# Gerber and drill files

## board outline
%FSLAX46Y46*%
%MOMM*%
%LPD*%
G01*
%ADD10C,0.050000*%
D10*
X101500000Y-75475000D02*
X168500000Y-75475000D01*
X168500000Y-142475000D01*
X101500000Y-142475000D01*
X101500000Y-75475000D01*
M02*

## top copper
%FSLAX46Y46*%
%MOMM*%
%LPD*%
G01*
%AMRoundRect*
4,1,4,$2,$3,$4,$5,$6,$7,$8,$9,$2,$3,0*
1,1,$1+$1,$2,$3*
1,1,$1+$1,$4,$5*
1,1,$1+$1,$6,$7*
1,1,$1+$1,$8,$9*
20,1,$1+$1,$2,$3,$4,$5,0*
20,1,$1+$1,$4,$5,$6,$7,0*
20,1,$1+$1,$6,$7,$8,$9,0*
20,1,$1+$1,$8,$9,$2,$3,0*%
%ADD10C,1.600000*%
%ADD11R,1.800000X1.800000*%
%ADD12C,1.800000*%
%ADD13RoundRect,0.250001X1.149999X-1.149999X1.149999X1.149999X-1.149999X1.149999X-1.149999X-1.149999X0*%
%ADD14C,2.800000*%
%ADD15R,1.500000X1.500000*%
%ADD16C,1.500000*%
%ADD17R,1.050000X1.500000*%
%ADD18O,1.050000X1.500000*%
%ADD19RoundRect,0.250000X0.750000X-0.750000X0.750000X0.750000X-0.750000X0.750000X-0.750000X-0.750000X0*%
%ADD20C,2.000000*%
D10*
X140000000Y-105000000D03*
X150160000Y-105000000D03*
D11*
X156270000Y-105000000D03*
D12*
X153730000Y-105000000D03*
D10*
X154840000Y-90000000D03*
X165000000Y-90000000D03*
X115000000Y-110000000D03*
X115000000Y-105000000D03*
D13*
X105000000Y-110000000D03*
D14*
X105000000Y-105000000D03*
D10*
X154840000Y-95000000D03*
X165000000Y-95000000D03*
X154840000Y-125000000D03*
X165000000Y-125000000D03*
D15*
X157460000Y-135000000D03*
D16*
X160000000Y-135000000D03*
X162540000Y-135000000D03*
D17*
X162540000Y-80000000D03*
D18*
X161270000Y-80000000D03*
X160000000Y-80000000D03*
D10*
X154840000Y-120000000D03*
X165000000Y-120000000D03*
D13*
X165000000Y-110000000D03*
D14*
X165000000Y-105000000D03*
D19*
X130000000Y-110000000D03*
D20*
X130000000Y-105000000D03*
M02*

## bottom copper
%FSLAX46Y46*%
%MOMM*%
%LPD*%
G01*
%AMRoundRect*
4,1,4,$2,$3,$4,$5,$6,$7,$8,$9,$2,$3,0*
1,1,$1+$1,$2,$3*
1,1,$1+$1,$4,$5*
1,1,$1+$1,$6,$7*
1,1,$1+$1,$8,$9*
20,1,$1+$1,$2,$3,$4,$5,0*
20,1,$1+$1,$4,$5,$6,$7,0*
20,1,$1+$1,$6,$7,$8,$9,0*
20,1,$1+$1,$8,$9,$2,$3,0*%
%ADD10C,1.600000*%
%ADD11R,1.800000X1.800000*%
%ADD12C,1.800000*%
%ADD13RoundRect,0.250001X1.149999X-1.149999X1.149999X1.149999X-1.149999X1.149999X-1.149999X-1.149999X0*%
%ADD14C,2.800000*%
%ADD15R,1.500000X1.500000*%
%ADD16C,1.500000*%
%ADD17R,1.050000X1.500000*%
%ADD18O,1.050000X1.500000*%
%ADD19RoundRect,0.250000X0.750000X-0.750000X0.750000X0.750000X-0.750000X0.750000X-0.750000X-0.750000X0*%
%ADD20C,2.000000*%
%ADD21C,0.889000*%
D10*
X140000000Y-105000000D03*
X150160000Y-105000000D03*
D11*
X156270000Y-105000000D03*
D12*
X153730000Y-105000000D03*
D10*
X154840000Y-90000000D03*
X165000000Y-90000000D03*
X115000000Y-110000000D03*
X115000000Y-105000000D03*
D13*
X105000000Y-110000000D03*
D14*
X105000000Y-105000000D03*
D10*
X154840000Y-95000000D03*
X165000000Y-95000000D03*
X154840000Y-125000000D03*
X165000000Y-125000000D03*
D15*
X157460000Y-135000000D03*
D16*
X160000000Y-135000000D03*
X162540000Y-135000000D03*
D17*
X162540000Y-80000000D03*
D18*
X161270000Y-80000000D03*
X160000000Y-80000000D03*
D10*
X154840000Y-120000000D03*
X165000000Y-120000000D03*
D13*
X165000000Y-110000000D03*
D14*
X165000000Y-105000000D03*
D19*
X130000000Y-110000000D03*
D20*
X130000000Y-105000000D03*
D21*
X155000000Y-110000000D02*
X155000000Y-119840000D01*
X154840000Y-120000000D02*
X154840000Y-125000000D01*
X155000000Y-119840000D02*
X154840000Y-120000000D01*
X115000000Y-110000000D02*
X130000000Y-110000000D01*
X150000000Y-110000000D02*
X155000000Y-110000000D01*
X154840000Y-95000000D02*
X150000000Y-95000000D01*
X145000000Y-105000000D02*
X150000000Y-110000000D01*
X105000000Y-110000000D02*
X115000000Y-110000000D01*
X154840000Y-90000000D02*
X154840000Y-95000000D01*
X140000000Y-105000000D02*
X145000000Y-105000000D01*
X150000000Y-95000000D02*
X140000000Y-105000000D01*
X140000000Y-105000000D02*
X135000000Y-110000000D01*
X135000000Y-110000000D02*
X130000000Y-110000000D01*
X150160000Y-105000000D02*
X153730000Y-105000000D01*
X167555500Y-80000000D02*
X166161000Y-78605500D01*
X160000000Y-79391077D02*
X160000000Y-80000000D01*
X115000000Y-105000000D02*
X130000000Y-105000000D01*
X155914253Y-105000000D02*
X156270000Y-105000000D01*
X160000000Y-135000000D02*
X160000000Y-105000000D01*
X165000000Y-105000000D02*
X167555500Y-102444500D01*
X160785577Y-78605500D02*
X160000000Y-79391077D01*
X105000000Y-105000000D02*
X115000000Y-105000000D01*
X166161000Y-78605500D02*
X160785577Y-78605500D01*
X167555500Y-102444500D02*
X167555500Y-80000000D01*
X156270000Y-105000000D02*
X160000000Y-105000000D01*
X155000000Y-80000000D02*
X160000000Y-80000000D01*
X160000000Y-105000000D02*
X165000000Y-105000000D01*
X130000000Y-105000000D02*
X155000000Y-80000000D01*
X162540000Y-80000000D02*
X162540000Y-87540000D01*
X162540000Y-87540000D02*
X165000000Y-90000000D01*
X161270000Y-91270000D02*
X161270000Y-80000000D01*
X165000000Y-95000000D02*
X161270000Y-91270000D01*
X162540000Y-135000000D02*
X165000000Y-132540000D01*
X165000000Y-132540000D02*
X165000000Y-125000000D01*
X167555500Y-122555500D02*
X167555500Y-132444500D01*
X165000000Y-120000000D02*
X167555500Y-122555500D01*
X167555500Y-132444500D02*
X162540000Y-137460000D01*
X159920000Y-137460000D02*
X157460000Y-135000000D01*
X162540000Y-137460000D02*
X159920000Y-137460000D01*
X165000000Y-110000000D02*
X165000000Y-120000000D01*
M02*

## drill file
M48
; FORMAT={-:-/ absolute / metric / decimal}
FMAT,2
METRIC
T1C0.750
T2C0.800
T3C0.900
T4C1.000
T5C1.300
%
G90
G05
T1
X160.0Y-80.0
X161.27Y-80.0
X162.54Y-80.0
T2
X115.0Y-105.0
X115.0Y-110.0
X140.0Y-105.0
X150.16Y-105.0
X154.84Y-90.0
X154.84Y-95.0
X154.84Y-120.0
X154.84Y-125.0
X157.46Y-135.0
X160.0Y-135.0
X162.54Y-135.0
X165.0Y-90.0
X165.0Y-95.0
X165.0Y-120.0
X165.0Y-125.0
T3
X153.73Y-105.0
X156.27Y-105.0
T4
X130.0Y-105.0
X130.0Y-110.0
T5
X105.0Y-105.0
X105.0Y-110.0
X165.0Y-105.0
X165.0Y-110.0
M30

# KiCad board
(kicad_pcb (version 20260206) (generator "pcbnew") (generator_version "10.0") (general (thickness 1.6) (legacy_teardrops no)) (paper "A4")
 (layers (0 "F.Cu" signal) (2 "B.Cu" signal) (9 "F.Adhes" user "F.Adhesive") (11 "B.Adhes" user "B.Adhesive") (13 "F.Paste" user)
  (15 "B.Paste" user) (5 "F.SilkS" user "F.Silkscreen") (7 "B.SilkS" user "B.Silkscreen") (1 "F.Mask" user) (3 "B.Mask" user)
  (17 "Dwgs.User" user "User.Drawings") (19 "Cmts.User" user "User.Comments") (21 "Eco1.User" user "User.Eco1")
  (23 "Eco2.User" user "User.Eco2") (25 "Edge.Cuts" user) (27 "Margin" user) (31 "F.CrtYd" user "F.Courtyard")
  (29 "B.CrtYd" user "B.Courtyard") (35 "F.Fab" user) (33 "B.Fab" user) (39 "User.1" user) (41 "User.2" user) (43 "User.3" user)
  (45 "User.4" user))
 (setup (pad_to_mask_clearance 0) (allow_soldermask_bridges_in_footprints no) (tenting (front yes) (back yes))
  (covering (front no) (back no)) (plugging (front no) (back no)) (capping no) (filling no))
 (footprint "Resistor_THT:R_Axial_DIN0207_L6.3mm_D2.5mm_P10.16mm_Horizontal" (layer "F.Cu") (at 140 105)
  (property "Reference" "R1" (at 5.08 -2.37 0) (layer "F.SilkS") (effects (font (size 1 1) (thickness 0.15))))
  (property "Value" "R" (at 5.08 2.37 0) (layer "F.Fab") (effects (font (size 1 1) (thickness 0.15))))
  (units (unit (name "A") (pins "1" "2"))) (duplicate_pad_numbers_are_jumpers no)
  (pad "1" thru_hole circle (at 0 0) (size 1.6 1.6) (drill 0.8) (layers "*.Cu" "*.Mask") (remove_unused_layers no) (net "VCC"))
  (pad "2" thru_hole circle (at 10.16 0) (size 1.6 1.6) (drill 0.8) (layers "*.Cu" "*.Mask") (remove_unused_layers no) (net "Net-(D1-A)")))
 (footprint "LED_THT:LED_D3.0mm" (layer "F.Cu") (at 156.27 105 180)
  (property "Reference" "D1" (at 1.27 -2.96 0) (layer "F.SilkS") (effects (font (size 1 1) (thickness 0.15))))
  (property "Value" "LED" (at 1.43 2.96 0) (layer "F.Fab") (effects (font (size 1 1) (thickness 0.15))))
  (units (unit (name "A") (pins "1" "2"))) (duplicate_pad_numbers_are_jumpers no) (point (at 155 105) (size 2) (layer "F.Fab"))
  (pad "1" thru_hole rect (at 0 0 180) (size 1.8 1.8) (drill 0.9) (layers "*.Cu" "*.Mask") (remove_unused_layers no) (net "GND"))
  (pad "2" thru_hole circle (at 2.54 0 180) (size 1.8 1.8) (drill 0.9) (layers "*.Cu" "*.Mask") (remove_unused_layers no) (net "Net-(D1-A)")))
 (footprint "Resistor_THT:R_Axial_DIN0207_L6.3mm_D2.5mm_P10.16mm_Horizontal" (layer "F.Cu") (at 154.84 90)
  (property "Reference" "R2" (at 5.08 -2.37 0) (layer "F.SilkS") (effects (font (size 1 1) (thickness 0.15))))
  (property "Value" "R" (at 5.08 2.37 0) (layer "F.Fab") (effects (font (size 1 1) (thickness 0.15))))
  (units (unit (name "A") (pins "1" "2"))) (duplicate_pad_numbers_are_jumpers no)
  (pad "1" thru_hole circle (at 0 0) (size 1.6 1.6) (drill 0.8) (layers "*.Cu" "*.Mask") (remove_unused_layers no) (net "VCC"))
  (pad "2" thru_hole circle (at 10.16 0) (size 1.6 1.6) (drill 0.8) (layers "*.Cu" "*.Mask") (remove_unused_layers no) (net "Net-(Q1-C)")))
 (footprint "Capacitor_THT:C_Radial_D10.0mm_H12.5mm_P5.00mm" (layer "F.Cu") (at 115 110 90)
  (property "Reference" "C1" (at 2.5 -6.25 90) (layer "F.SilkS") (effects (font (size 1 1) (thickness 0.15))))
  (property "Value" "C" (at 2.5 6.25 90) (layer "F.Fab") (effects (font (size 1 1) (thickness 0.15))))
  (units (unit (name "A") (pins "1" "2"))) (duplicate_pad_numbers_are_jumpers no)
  (pad "1" thru_hole circle (at 0 0 90) (size 1.6 1.6) (drill 0.8) (layers "*.Cu" "*.Mask") (remove_unused_layers no) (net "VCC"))
  (pad "2" thru_hole circle (at 5 0 90) (size 1.6 1.6) (drill 0.8) (layers "*.Cu" "*.Mask") (remove_unused_layers no) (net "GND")))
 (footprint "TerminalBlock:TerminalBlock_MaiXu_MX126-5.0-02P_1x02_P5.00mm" (layer "F.Cu") (at 105 110 90)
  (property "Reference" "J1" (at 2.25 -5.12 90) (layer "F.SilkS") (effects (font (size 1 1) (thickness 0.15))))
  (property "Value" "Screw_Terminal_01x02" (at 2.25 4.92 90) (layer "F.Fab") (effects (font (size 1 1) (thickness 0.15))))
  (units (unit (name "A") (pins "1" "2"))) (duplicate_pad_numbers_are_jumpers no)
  (pad "1" thru_hole roundrect (at 0 0 90) (size 2.8 2.8) (drill 1.3) (layers "*.Cu" "*.Mask") (remove_unused_layers no)
   (roundrect_rratio 0.089286) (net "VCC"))
  (pad "2" thru_hole circle (at 5 0 90) (size 2.8 2.8) (drill 1.3) (layers "*.Cu" "*.Mask") (remove_unused_layers no) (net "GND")))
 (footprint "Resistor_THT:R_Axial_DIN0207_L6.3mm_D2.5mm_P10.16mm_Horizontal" (layer "F.Cu") (at 154.84 95)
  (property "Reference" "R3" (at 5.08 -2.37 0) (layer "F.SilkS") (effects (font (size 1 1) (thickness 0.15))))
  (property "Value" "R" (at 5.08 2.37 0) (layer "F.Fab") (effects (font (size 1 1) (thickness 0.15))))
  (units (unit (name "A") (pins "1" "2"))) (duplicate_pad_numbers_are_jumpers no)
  (pad "1" thru_hole circle (at 0 0) (size 1.6 1.6) (drill 0.8) (layers "*.Cu" "*.Mask") (remove_unused_layers no) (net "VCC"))
  (pad "2" thru_hole circle (at 10.16 0) (size 1.6 1.6) (drill 0.8) (layers "*.Cu" "*.Mask") (remove_unused_layers no) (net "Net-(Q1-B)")))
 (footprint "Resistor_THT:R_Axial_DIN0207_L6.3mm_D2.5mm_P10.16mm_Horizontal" (layer "F.Cu") (at 154.84 125)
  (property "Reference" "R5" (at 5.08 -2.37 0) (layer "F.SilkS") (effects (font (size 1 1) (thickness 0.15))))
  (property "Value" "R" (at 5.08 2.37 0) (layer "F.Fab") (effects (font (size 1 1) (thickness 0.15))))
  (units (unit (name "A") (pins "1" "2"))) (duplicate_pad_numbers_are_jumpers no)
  (pad "1" thru_hole circle (at 0 0) (size 1.6 1.6) (drill 0.8) (layers "*.Cu" "*.Mask") (remove_unused_layers no) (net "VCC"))
  (pad "2" thru_hole circle (at 10.16 0) (size 1.6 1.6) (drill 0.8) (layers "*.Cu" "*.Mask") (remove_unused_layers no) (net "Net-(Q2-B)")))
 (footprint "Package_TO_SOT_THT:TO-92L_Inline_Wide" (layer "F.Cu") (at 157.46 135)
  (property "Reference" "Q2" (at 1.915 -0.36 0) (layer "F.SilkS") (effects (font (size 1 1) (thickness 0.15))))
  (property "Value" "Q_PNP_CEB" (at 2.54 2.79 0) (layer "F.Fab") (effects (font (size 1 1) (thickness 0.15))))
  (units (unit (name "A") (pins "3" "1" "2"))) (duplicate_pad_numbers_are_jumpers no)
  (pad "1" thru_hole rect (at 0 0) (size 1.5 1.5) (drill 0.8) (layers "*.Cu" "*.Mask") (remove_unused_layers no) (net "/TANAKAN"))
  (pad "2" thru_hole circle (at 2.54 0) (size 1.5 1.5) (drill 0.8) (layers "*.Cu" "*.Mask") (remove_unused_layers no) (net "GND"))
  (pad "3" thru_hole circle (at 5.08 0) (size 1.5 1.5) (drill 0.8) (layers "*.Cu" "*.Mask") (remove_unused_layers no) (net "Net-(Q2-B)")))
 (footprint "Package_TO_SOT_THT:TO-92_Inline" (layer "F.Cu") (at 162.54 80 180)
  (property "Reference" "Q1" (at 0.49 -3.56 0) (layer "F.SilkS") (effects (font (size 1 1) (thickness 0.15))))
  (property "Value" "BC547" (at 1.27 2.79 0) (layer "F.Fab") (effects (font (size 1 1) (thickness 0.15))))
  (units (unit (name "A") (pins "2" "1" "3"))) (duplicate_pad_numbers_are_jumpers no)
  (pad "1" thru_hole rect (at 0 0 180) (size 1.05 1.5) (drill 0.75) (layers "*.Cu" "*.Mask") (remove_unused_layers no) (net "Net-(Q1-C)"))
  (pad "2" thru_hole oval (at 1.27 0 180) (size 1.05 1.5) (drill 0.75) (layers "*.Cu" "*.Mask") (remove_unused_layers no) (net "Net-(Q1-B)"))
  (pad "3" thru_hole oval (at 2.54 0 180) (size 1.05 1.5) (drill 0.75) (layers "*.Cu" "*.Mask") (remove_unused_layers no) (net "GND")))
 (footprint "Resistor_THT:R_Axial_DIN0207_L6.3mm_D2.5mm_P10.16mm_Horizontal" (layer "F.Cu") (at 154.84 120)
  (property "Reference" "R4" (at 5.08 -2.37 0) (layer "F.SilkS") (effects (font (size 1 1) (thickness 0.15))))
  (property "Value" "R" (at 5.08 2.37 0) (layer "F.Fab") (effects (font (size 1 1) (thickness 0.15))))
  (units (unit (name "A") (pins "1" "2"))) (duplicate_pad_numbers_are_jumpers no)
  (pad "1" thru_hole circle (at 0 0) (size 1.6 1.6) (drill 0.8) (layers "*.Cu" "*.Mask") (remove_unused_layers no) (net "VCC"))
  (pad "2" thru_hole circle (at 10.16 0) (size 1.6 1.6) (drill 0.8) (layers "*.Cu" "*.Mask") (remove_unused_layers no) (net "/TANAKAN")))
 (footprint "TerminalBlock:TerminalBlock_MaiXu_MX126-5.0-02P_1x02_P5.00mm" (layer "F.Cu") (at 165 110 90)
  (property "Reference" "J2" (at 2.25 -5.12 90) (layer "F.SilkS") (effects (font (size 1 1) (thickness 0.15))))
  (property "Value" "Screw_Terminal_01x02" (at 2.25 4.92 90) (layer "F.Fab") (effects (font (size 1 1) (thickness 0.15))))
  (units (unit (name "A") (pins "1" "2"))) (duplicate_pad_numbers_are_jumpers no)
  (pad "1" thru_hole roundrect (at 0 0 90) (size 2.8 2.8) (drill 1.3) (layers "*.Cu" "*.Mask") (remove_unused_layers no)
   (roundrect_rratio 0.089286) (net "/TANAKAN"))
  (pad "2" thru_hole circle (at 5 0 90) (size 2.8 2.8) (drill 1.3) (layers "*.Cu" "*.Mask") (remove_unused_layers no) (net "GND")))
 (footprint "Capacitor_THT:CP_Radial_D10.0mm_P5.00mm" (layer "F.Cu") (at 130 110 90)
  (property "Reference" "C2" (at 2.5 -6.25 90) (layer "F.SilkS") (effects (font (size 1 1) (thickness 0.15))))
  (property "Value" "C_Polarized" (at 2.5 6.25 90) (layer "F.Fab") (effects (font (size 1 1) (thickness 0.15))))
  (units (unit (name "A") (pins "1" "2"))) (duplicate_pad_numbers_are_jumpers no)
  (pad "1" thru_hole roundrect (at 0 0 90) (size 2 2) (drill 1) (layers "*.Cu" "*.Mask") (remove_unused_layers no) (roundrect_rratio 0.125)
   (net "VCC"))
  (pad "2" thru_hole circle (at 5 0 90) (size 2 2) (drill 1) (layers "*.Cu" "*.Mask") (remove_unused_layers no) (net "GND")))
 (gr_rect (start 101.5 75.475) (end 168.5 142.475) (stroke (width 0.05) (type default)) (fill no) (layer "Edge.Cuts"))
 (segment (start 155 110) (end 155 119.84) (width 0.889) (layer "B.Cu") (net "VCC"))
 (segment (start 154.84 120) (end 154.84 125) (width 0.889) (layer "B.Cu") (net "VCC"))
 (segment (start 155 119.84) (end 154.84 120) (width 0.889) (layer "B.Cu") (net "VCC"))
 (segment (start 115 110) (end 130 110) (width 0.889) (layer "B.Cu") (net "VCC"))
 (segment (start 150 110) (end 155 110) (width 0.889) (layer "B.Cu") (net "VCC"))
 (segment (start 154.84 95) (end 150 95) (width 0.889) (layer "B.Cu") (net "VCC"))
 (segment (start 145 105) (end 150 110) (width 0.889) (layer "B.Cu") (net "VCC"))
 (segment (start 105 110) (end 115 110) (width 0.889) (layer "B.Cu") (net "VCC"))
 (segment (start 154.84 90) (end 154.84 95) (width 0.889) (layer "B.Cu") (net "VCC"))
 (segment (start 140 105) (end 145 105) (width 0.889) (layer "B.Cu") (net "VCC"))
 (segment (start 150 95) (end 140 105) (width 0.889) (layer "B.Cu") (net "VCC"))
 (segment (start 140 105) (end 135 110) (width 0.889) (layer "B.Cu") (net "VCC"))
 (segment (start 135 110) (end 130 110) (width 0.889) (layer "B.Cu") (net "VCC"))
 (segment (start 150.16 105) (end 153.73 105) (width 0.889) (layer "B.Cu") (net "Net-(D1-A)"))
 (segment (start 167.5555 80) (end 166.161 78.6055) (width 0.889) (layer "B.Cu") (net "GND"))
 (segment (start 160 79.391077) (end 160 80) (width 0.889) (layer "B.Cu") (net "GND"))
 (segment (start 115 105) (end 130 105) (width 0.889) (layer "B.Cu") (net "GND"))
 (segment (start 155.914253 105) (end 156.27 105) (width 0.889) (layer "B.Cu") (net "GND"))
 (segment (start 160 135) (end 160 105) (width 0.889) (layer "B.Cu") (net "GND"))
 (segment (start 165 105) (end 167.5555 102.4445) (width 0.889) (layer "B.Cu") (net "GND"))
 (segment (start 160.785577 78.6055) (end 160 79.391077) (width 0.889) (layer "B.Cu") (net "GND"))
 (segment (start 105 105) (end 115 105) (width 0.889) (layer "B.Cu") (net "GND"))
 (segment (start 166.161 78.6055) (end 160.785577 78.6055) (width 0.889) (layer "B.Cu") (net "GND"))
 (segment (start 167.5555 102.4445) (end 167.5555 80) (width 0.889) (layer "B.Cu") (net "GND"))
 (segment (start 156.27 105) (end 160 105) (width 0.889) (layer "B.Cu") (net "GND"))
 (segment (start 155 80) (end 160 80) (width 0.889) (layer "B.Cu") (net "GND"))
 (segment (start 160 105) (end 165 105) (width 0.889) (layer "B.Cu") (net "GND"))
 (segment (start 130 105) (end 155 80) (width 0.889) (layer "B.Cu") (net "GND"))
 (segment (start 162.54 80) (end 162.54 87.54) (width 0.889) (layer "B.Cu") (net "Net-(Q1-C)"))
 (segment (start 162.54 87.54) (end 165 90) (width 0.889) (layer "B.Cu") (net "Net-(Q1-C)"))
 (segment (start 161.27 91.27) (end 161.27 80) (width 0.889) (layer "B.Cu") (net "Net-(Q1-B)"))
 (segment (start 165 95) (end 161.27 91.27) (width 0.889) (layer "B.Cu") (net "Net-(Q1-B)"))
 (segment (start 162.54 135) (end 165 132.54) (width 0.889) (layer "B.Cu") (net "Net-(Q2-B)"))
 (segment (start 165 132.54) (end 165 125) (width 0.889) (layer "B.Cu") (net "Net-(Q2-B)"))
 (segment (start 167.5555 122.5555) (end 167.5555 132.4445) (width 0.889) (layer "B.Cu") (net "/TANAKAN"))
 (segment (start 165 120) (end 167.5555 122.5555) (width 0.889) (layer "B.Cu") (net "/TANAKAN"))
 (segment (start 167.5555 132.4445) (end 162.54 137.46) (width 0.889) (layer "B.Cu") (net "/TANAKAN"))
 (segment (start 159.92 137.46) (end 157.46 135) (width 0.889) (layer "B.Cu") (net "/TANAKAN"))
 (segment (start 162.54 137.46) (end 159.92 137.46) (width 0.889) (layer "B.Cu") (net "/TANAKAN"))
 (segment (start 165 110) (end 165 120) (width 0.889) (layer "B.Cu") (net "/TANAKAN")))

